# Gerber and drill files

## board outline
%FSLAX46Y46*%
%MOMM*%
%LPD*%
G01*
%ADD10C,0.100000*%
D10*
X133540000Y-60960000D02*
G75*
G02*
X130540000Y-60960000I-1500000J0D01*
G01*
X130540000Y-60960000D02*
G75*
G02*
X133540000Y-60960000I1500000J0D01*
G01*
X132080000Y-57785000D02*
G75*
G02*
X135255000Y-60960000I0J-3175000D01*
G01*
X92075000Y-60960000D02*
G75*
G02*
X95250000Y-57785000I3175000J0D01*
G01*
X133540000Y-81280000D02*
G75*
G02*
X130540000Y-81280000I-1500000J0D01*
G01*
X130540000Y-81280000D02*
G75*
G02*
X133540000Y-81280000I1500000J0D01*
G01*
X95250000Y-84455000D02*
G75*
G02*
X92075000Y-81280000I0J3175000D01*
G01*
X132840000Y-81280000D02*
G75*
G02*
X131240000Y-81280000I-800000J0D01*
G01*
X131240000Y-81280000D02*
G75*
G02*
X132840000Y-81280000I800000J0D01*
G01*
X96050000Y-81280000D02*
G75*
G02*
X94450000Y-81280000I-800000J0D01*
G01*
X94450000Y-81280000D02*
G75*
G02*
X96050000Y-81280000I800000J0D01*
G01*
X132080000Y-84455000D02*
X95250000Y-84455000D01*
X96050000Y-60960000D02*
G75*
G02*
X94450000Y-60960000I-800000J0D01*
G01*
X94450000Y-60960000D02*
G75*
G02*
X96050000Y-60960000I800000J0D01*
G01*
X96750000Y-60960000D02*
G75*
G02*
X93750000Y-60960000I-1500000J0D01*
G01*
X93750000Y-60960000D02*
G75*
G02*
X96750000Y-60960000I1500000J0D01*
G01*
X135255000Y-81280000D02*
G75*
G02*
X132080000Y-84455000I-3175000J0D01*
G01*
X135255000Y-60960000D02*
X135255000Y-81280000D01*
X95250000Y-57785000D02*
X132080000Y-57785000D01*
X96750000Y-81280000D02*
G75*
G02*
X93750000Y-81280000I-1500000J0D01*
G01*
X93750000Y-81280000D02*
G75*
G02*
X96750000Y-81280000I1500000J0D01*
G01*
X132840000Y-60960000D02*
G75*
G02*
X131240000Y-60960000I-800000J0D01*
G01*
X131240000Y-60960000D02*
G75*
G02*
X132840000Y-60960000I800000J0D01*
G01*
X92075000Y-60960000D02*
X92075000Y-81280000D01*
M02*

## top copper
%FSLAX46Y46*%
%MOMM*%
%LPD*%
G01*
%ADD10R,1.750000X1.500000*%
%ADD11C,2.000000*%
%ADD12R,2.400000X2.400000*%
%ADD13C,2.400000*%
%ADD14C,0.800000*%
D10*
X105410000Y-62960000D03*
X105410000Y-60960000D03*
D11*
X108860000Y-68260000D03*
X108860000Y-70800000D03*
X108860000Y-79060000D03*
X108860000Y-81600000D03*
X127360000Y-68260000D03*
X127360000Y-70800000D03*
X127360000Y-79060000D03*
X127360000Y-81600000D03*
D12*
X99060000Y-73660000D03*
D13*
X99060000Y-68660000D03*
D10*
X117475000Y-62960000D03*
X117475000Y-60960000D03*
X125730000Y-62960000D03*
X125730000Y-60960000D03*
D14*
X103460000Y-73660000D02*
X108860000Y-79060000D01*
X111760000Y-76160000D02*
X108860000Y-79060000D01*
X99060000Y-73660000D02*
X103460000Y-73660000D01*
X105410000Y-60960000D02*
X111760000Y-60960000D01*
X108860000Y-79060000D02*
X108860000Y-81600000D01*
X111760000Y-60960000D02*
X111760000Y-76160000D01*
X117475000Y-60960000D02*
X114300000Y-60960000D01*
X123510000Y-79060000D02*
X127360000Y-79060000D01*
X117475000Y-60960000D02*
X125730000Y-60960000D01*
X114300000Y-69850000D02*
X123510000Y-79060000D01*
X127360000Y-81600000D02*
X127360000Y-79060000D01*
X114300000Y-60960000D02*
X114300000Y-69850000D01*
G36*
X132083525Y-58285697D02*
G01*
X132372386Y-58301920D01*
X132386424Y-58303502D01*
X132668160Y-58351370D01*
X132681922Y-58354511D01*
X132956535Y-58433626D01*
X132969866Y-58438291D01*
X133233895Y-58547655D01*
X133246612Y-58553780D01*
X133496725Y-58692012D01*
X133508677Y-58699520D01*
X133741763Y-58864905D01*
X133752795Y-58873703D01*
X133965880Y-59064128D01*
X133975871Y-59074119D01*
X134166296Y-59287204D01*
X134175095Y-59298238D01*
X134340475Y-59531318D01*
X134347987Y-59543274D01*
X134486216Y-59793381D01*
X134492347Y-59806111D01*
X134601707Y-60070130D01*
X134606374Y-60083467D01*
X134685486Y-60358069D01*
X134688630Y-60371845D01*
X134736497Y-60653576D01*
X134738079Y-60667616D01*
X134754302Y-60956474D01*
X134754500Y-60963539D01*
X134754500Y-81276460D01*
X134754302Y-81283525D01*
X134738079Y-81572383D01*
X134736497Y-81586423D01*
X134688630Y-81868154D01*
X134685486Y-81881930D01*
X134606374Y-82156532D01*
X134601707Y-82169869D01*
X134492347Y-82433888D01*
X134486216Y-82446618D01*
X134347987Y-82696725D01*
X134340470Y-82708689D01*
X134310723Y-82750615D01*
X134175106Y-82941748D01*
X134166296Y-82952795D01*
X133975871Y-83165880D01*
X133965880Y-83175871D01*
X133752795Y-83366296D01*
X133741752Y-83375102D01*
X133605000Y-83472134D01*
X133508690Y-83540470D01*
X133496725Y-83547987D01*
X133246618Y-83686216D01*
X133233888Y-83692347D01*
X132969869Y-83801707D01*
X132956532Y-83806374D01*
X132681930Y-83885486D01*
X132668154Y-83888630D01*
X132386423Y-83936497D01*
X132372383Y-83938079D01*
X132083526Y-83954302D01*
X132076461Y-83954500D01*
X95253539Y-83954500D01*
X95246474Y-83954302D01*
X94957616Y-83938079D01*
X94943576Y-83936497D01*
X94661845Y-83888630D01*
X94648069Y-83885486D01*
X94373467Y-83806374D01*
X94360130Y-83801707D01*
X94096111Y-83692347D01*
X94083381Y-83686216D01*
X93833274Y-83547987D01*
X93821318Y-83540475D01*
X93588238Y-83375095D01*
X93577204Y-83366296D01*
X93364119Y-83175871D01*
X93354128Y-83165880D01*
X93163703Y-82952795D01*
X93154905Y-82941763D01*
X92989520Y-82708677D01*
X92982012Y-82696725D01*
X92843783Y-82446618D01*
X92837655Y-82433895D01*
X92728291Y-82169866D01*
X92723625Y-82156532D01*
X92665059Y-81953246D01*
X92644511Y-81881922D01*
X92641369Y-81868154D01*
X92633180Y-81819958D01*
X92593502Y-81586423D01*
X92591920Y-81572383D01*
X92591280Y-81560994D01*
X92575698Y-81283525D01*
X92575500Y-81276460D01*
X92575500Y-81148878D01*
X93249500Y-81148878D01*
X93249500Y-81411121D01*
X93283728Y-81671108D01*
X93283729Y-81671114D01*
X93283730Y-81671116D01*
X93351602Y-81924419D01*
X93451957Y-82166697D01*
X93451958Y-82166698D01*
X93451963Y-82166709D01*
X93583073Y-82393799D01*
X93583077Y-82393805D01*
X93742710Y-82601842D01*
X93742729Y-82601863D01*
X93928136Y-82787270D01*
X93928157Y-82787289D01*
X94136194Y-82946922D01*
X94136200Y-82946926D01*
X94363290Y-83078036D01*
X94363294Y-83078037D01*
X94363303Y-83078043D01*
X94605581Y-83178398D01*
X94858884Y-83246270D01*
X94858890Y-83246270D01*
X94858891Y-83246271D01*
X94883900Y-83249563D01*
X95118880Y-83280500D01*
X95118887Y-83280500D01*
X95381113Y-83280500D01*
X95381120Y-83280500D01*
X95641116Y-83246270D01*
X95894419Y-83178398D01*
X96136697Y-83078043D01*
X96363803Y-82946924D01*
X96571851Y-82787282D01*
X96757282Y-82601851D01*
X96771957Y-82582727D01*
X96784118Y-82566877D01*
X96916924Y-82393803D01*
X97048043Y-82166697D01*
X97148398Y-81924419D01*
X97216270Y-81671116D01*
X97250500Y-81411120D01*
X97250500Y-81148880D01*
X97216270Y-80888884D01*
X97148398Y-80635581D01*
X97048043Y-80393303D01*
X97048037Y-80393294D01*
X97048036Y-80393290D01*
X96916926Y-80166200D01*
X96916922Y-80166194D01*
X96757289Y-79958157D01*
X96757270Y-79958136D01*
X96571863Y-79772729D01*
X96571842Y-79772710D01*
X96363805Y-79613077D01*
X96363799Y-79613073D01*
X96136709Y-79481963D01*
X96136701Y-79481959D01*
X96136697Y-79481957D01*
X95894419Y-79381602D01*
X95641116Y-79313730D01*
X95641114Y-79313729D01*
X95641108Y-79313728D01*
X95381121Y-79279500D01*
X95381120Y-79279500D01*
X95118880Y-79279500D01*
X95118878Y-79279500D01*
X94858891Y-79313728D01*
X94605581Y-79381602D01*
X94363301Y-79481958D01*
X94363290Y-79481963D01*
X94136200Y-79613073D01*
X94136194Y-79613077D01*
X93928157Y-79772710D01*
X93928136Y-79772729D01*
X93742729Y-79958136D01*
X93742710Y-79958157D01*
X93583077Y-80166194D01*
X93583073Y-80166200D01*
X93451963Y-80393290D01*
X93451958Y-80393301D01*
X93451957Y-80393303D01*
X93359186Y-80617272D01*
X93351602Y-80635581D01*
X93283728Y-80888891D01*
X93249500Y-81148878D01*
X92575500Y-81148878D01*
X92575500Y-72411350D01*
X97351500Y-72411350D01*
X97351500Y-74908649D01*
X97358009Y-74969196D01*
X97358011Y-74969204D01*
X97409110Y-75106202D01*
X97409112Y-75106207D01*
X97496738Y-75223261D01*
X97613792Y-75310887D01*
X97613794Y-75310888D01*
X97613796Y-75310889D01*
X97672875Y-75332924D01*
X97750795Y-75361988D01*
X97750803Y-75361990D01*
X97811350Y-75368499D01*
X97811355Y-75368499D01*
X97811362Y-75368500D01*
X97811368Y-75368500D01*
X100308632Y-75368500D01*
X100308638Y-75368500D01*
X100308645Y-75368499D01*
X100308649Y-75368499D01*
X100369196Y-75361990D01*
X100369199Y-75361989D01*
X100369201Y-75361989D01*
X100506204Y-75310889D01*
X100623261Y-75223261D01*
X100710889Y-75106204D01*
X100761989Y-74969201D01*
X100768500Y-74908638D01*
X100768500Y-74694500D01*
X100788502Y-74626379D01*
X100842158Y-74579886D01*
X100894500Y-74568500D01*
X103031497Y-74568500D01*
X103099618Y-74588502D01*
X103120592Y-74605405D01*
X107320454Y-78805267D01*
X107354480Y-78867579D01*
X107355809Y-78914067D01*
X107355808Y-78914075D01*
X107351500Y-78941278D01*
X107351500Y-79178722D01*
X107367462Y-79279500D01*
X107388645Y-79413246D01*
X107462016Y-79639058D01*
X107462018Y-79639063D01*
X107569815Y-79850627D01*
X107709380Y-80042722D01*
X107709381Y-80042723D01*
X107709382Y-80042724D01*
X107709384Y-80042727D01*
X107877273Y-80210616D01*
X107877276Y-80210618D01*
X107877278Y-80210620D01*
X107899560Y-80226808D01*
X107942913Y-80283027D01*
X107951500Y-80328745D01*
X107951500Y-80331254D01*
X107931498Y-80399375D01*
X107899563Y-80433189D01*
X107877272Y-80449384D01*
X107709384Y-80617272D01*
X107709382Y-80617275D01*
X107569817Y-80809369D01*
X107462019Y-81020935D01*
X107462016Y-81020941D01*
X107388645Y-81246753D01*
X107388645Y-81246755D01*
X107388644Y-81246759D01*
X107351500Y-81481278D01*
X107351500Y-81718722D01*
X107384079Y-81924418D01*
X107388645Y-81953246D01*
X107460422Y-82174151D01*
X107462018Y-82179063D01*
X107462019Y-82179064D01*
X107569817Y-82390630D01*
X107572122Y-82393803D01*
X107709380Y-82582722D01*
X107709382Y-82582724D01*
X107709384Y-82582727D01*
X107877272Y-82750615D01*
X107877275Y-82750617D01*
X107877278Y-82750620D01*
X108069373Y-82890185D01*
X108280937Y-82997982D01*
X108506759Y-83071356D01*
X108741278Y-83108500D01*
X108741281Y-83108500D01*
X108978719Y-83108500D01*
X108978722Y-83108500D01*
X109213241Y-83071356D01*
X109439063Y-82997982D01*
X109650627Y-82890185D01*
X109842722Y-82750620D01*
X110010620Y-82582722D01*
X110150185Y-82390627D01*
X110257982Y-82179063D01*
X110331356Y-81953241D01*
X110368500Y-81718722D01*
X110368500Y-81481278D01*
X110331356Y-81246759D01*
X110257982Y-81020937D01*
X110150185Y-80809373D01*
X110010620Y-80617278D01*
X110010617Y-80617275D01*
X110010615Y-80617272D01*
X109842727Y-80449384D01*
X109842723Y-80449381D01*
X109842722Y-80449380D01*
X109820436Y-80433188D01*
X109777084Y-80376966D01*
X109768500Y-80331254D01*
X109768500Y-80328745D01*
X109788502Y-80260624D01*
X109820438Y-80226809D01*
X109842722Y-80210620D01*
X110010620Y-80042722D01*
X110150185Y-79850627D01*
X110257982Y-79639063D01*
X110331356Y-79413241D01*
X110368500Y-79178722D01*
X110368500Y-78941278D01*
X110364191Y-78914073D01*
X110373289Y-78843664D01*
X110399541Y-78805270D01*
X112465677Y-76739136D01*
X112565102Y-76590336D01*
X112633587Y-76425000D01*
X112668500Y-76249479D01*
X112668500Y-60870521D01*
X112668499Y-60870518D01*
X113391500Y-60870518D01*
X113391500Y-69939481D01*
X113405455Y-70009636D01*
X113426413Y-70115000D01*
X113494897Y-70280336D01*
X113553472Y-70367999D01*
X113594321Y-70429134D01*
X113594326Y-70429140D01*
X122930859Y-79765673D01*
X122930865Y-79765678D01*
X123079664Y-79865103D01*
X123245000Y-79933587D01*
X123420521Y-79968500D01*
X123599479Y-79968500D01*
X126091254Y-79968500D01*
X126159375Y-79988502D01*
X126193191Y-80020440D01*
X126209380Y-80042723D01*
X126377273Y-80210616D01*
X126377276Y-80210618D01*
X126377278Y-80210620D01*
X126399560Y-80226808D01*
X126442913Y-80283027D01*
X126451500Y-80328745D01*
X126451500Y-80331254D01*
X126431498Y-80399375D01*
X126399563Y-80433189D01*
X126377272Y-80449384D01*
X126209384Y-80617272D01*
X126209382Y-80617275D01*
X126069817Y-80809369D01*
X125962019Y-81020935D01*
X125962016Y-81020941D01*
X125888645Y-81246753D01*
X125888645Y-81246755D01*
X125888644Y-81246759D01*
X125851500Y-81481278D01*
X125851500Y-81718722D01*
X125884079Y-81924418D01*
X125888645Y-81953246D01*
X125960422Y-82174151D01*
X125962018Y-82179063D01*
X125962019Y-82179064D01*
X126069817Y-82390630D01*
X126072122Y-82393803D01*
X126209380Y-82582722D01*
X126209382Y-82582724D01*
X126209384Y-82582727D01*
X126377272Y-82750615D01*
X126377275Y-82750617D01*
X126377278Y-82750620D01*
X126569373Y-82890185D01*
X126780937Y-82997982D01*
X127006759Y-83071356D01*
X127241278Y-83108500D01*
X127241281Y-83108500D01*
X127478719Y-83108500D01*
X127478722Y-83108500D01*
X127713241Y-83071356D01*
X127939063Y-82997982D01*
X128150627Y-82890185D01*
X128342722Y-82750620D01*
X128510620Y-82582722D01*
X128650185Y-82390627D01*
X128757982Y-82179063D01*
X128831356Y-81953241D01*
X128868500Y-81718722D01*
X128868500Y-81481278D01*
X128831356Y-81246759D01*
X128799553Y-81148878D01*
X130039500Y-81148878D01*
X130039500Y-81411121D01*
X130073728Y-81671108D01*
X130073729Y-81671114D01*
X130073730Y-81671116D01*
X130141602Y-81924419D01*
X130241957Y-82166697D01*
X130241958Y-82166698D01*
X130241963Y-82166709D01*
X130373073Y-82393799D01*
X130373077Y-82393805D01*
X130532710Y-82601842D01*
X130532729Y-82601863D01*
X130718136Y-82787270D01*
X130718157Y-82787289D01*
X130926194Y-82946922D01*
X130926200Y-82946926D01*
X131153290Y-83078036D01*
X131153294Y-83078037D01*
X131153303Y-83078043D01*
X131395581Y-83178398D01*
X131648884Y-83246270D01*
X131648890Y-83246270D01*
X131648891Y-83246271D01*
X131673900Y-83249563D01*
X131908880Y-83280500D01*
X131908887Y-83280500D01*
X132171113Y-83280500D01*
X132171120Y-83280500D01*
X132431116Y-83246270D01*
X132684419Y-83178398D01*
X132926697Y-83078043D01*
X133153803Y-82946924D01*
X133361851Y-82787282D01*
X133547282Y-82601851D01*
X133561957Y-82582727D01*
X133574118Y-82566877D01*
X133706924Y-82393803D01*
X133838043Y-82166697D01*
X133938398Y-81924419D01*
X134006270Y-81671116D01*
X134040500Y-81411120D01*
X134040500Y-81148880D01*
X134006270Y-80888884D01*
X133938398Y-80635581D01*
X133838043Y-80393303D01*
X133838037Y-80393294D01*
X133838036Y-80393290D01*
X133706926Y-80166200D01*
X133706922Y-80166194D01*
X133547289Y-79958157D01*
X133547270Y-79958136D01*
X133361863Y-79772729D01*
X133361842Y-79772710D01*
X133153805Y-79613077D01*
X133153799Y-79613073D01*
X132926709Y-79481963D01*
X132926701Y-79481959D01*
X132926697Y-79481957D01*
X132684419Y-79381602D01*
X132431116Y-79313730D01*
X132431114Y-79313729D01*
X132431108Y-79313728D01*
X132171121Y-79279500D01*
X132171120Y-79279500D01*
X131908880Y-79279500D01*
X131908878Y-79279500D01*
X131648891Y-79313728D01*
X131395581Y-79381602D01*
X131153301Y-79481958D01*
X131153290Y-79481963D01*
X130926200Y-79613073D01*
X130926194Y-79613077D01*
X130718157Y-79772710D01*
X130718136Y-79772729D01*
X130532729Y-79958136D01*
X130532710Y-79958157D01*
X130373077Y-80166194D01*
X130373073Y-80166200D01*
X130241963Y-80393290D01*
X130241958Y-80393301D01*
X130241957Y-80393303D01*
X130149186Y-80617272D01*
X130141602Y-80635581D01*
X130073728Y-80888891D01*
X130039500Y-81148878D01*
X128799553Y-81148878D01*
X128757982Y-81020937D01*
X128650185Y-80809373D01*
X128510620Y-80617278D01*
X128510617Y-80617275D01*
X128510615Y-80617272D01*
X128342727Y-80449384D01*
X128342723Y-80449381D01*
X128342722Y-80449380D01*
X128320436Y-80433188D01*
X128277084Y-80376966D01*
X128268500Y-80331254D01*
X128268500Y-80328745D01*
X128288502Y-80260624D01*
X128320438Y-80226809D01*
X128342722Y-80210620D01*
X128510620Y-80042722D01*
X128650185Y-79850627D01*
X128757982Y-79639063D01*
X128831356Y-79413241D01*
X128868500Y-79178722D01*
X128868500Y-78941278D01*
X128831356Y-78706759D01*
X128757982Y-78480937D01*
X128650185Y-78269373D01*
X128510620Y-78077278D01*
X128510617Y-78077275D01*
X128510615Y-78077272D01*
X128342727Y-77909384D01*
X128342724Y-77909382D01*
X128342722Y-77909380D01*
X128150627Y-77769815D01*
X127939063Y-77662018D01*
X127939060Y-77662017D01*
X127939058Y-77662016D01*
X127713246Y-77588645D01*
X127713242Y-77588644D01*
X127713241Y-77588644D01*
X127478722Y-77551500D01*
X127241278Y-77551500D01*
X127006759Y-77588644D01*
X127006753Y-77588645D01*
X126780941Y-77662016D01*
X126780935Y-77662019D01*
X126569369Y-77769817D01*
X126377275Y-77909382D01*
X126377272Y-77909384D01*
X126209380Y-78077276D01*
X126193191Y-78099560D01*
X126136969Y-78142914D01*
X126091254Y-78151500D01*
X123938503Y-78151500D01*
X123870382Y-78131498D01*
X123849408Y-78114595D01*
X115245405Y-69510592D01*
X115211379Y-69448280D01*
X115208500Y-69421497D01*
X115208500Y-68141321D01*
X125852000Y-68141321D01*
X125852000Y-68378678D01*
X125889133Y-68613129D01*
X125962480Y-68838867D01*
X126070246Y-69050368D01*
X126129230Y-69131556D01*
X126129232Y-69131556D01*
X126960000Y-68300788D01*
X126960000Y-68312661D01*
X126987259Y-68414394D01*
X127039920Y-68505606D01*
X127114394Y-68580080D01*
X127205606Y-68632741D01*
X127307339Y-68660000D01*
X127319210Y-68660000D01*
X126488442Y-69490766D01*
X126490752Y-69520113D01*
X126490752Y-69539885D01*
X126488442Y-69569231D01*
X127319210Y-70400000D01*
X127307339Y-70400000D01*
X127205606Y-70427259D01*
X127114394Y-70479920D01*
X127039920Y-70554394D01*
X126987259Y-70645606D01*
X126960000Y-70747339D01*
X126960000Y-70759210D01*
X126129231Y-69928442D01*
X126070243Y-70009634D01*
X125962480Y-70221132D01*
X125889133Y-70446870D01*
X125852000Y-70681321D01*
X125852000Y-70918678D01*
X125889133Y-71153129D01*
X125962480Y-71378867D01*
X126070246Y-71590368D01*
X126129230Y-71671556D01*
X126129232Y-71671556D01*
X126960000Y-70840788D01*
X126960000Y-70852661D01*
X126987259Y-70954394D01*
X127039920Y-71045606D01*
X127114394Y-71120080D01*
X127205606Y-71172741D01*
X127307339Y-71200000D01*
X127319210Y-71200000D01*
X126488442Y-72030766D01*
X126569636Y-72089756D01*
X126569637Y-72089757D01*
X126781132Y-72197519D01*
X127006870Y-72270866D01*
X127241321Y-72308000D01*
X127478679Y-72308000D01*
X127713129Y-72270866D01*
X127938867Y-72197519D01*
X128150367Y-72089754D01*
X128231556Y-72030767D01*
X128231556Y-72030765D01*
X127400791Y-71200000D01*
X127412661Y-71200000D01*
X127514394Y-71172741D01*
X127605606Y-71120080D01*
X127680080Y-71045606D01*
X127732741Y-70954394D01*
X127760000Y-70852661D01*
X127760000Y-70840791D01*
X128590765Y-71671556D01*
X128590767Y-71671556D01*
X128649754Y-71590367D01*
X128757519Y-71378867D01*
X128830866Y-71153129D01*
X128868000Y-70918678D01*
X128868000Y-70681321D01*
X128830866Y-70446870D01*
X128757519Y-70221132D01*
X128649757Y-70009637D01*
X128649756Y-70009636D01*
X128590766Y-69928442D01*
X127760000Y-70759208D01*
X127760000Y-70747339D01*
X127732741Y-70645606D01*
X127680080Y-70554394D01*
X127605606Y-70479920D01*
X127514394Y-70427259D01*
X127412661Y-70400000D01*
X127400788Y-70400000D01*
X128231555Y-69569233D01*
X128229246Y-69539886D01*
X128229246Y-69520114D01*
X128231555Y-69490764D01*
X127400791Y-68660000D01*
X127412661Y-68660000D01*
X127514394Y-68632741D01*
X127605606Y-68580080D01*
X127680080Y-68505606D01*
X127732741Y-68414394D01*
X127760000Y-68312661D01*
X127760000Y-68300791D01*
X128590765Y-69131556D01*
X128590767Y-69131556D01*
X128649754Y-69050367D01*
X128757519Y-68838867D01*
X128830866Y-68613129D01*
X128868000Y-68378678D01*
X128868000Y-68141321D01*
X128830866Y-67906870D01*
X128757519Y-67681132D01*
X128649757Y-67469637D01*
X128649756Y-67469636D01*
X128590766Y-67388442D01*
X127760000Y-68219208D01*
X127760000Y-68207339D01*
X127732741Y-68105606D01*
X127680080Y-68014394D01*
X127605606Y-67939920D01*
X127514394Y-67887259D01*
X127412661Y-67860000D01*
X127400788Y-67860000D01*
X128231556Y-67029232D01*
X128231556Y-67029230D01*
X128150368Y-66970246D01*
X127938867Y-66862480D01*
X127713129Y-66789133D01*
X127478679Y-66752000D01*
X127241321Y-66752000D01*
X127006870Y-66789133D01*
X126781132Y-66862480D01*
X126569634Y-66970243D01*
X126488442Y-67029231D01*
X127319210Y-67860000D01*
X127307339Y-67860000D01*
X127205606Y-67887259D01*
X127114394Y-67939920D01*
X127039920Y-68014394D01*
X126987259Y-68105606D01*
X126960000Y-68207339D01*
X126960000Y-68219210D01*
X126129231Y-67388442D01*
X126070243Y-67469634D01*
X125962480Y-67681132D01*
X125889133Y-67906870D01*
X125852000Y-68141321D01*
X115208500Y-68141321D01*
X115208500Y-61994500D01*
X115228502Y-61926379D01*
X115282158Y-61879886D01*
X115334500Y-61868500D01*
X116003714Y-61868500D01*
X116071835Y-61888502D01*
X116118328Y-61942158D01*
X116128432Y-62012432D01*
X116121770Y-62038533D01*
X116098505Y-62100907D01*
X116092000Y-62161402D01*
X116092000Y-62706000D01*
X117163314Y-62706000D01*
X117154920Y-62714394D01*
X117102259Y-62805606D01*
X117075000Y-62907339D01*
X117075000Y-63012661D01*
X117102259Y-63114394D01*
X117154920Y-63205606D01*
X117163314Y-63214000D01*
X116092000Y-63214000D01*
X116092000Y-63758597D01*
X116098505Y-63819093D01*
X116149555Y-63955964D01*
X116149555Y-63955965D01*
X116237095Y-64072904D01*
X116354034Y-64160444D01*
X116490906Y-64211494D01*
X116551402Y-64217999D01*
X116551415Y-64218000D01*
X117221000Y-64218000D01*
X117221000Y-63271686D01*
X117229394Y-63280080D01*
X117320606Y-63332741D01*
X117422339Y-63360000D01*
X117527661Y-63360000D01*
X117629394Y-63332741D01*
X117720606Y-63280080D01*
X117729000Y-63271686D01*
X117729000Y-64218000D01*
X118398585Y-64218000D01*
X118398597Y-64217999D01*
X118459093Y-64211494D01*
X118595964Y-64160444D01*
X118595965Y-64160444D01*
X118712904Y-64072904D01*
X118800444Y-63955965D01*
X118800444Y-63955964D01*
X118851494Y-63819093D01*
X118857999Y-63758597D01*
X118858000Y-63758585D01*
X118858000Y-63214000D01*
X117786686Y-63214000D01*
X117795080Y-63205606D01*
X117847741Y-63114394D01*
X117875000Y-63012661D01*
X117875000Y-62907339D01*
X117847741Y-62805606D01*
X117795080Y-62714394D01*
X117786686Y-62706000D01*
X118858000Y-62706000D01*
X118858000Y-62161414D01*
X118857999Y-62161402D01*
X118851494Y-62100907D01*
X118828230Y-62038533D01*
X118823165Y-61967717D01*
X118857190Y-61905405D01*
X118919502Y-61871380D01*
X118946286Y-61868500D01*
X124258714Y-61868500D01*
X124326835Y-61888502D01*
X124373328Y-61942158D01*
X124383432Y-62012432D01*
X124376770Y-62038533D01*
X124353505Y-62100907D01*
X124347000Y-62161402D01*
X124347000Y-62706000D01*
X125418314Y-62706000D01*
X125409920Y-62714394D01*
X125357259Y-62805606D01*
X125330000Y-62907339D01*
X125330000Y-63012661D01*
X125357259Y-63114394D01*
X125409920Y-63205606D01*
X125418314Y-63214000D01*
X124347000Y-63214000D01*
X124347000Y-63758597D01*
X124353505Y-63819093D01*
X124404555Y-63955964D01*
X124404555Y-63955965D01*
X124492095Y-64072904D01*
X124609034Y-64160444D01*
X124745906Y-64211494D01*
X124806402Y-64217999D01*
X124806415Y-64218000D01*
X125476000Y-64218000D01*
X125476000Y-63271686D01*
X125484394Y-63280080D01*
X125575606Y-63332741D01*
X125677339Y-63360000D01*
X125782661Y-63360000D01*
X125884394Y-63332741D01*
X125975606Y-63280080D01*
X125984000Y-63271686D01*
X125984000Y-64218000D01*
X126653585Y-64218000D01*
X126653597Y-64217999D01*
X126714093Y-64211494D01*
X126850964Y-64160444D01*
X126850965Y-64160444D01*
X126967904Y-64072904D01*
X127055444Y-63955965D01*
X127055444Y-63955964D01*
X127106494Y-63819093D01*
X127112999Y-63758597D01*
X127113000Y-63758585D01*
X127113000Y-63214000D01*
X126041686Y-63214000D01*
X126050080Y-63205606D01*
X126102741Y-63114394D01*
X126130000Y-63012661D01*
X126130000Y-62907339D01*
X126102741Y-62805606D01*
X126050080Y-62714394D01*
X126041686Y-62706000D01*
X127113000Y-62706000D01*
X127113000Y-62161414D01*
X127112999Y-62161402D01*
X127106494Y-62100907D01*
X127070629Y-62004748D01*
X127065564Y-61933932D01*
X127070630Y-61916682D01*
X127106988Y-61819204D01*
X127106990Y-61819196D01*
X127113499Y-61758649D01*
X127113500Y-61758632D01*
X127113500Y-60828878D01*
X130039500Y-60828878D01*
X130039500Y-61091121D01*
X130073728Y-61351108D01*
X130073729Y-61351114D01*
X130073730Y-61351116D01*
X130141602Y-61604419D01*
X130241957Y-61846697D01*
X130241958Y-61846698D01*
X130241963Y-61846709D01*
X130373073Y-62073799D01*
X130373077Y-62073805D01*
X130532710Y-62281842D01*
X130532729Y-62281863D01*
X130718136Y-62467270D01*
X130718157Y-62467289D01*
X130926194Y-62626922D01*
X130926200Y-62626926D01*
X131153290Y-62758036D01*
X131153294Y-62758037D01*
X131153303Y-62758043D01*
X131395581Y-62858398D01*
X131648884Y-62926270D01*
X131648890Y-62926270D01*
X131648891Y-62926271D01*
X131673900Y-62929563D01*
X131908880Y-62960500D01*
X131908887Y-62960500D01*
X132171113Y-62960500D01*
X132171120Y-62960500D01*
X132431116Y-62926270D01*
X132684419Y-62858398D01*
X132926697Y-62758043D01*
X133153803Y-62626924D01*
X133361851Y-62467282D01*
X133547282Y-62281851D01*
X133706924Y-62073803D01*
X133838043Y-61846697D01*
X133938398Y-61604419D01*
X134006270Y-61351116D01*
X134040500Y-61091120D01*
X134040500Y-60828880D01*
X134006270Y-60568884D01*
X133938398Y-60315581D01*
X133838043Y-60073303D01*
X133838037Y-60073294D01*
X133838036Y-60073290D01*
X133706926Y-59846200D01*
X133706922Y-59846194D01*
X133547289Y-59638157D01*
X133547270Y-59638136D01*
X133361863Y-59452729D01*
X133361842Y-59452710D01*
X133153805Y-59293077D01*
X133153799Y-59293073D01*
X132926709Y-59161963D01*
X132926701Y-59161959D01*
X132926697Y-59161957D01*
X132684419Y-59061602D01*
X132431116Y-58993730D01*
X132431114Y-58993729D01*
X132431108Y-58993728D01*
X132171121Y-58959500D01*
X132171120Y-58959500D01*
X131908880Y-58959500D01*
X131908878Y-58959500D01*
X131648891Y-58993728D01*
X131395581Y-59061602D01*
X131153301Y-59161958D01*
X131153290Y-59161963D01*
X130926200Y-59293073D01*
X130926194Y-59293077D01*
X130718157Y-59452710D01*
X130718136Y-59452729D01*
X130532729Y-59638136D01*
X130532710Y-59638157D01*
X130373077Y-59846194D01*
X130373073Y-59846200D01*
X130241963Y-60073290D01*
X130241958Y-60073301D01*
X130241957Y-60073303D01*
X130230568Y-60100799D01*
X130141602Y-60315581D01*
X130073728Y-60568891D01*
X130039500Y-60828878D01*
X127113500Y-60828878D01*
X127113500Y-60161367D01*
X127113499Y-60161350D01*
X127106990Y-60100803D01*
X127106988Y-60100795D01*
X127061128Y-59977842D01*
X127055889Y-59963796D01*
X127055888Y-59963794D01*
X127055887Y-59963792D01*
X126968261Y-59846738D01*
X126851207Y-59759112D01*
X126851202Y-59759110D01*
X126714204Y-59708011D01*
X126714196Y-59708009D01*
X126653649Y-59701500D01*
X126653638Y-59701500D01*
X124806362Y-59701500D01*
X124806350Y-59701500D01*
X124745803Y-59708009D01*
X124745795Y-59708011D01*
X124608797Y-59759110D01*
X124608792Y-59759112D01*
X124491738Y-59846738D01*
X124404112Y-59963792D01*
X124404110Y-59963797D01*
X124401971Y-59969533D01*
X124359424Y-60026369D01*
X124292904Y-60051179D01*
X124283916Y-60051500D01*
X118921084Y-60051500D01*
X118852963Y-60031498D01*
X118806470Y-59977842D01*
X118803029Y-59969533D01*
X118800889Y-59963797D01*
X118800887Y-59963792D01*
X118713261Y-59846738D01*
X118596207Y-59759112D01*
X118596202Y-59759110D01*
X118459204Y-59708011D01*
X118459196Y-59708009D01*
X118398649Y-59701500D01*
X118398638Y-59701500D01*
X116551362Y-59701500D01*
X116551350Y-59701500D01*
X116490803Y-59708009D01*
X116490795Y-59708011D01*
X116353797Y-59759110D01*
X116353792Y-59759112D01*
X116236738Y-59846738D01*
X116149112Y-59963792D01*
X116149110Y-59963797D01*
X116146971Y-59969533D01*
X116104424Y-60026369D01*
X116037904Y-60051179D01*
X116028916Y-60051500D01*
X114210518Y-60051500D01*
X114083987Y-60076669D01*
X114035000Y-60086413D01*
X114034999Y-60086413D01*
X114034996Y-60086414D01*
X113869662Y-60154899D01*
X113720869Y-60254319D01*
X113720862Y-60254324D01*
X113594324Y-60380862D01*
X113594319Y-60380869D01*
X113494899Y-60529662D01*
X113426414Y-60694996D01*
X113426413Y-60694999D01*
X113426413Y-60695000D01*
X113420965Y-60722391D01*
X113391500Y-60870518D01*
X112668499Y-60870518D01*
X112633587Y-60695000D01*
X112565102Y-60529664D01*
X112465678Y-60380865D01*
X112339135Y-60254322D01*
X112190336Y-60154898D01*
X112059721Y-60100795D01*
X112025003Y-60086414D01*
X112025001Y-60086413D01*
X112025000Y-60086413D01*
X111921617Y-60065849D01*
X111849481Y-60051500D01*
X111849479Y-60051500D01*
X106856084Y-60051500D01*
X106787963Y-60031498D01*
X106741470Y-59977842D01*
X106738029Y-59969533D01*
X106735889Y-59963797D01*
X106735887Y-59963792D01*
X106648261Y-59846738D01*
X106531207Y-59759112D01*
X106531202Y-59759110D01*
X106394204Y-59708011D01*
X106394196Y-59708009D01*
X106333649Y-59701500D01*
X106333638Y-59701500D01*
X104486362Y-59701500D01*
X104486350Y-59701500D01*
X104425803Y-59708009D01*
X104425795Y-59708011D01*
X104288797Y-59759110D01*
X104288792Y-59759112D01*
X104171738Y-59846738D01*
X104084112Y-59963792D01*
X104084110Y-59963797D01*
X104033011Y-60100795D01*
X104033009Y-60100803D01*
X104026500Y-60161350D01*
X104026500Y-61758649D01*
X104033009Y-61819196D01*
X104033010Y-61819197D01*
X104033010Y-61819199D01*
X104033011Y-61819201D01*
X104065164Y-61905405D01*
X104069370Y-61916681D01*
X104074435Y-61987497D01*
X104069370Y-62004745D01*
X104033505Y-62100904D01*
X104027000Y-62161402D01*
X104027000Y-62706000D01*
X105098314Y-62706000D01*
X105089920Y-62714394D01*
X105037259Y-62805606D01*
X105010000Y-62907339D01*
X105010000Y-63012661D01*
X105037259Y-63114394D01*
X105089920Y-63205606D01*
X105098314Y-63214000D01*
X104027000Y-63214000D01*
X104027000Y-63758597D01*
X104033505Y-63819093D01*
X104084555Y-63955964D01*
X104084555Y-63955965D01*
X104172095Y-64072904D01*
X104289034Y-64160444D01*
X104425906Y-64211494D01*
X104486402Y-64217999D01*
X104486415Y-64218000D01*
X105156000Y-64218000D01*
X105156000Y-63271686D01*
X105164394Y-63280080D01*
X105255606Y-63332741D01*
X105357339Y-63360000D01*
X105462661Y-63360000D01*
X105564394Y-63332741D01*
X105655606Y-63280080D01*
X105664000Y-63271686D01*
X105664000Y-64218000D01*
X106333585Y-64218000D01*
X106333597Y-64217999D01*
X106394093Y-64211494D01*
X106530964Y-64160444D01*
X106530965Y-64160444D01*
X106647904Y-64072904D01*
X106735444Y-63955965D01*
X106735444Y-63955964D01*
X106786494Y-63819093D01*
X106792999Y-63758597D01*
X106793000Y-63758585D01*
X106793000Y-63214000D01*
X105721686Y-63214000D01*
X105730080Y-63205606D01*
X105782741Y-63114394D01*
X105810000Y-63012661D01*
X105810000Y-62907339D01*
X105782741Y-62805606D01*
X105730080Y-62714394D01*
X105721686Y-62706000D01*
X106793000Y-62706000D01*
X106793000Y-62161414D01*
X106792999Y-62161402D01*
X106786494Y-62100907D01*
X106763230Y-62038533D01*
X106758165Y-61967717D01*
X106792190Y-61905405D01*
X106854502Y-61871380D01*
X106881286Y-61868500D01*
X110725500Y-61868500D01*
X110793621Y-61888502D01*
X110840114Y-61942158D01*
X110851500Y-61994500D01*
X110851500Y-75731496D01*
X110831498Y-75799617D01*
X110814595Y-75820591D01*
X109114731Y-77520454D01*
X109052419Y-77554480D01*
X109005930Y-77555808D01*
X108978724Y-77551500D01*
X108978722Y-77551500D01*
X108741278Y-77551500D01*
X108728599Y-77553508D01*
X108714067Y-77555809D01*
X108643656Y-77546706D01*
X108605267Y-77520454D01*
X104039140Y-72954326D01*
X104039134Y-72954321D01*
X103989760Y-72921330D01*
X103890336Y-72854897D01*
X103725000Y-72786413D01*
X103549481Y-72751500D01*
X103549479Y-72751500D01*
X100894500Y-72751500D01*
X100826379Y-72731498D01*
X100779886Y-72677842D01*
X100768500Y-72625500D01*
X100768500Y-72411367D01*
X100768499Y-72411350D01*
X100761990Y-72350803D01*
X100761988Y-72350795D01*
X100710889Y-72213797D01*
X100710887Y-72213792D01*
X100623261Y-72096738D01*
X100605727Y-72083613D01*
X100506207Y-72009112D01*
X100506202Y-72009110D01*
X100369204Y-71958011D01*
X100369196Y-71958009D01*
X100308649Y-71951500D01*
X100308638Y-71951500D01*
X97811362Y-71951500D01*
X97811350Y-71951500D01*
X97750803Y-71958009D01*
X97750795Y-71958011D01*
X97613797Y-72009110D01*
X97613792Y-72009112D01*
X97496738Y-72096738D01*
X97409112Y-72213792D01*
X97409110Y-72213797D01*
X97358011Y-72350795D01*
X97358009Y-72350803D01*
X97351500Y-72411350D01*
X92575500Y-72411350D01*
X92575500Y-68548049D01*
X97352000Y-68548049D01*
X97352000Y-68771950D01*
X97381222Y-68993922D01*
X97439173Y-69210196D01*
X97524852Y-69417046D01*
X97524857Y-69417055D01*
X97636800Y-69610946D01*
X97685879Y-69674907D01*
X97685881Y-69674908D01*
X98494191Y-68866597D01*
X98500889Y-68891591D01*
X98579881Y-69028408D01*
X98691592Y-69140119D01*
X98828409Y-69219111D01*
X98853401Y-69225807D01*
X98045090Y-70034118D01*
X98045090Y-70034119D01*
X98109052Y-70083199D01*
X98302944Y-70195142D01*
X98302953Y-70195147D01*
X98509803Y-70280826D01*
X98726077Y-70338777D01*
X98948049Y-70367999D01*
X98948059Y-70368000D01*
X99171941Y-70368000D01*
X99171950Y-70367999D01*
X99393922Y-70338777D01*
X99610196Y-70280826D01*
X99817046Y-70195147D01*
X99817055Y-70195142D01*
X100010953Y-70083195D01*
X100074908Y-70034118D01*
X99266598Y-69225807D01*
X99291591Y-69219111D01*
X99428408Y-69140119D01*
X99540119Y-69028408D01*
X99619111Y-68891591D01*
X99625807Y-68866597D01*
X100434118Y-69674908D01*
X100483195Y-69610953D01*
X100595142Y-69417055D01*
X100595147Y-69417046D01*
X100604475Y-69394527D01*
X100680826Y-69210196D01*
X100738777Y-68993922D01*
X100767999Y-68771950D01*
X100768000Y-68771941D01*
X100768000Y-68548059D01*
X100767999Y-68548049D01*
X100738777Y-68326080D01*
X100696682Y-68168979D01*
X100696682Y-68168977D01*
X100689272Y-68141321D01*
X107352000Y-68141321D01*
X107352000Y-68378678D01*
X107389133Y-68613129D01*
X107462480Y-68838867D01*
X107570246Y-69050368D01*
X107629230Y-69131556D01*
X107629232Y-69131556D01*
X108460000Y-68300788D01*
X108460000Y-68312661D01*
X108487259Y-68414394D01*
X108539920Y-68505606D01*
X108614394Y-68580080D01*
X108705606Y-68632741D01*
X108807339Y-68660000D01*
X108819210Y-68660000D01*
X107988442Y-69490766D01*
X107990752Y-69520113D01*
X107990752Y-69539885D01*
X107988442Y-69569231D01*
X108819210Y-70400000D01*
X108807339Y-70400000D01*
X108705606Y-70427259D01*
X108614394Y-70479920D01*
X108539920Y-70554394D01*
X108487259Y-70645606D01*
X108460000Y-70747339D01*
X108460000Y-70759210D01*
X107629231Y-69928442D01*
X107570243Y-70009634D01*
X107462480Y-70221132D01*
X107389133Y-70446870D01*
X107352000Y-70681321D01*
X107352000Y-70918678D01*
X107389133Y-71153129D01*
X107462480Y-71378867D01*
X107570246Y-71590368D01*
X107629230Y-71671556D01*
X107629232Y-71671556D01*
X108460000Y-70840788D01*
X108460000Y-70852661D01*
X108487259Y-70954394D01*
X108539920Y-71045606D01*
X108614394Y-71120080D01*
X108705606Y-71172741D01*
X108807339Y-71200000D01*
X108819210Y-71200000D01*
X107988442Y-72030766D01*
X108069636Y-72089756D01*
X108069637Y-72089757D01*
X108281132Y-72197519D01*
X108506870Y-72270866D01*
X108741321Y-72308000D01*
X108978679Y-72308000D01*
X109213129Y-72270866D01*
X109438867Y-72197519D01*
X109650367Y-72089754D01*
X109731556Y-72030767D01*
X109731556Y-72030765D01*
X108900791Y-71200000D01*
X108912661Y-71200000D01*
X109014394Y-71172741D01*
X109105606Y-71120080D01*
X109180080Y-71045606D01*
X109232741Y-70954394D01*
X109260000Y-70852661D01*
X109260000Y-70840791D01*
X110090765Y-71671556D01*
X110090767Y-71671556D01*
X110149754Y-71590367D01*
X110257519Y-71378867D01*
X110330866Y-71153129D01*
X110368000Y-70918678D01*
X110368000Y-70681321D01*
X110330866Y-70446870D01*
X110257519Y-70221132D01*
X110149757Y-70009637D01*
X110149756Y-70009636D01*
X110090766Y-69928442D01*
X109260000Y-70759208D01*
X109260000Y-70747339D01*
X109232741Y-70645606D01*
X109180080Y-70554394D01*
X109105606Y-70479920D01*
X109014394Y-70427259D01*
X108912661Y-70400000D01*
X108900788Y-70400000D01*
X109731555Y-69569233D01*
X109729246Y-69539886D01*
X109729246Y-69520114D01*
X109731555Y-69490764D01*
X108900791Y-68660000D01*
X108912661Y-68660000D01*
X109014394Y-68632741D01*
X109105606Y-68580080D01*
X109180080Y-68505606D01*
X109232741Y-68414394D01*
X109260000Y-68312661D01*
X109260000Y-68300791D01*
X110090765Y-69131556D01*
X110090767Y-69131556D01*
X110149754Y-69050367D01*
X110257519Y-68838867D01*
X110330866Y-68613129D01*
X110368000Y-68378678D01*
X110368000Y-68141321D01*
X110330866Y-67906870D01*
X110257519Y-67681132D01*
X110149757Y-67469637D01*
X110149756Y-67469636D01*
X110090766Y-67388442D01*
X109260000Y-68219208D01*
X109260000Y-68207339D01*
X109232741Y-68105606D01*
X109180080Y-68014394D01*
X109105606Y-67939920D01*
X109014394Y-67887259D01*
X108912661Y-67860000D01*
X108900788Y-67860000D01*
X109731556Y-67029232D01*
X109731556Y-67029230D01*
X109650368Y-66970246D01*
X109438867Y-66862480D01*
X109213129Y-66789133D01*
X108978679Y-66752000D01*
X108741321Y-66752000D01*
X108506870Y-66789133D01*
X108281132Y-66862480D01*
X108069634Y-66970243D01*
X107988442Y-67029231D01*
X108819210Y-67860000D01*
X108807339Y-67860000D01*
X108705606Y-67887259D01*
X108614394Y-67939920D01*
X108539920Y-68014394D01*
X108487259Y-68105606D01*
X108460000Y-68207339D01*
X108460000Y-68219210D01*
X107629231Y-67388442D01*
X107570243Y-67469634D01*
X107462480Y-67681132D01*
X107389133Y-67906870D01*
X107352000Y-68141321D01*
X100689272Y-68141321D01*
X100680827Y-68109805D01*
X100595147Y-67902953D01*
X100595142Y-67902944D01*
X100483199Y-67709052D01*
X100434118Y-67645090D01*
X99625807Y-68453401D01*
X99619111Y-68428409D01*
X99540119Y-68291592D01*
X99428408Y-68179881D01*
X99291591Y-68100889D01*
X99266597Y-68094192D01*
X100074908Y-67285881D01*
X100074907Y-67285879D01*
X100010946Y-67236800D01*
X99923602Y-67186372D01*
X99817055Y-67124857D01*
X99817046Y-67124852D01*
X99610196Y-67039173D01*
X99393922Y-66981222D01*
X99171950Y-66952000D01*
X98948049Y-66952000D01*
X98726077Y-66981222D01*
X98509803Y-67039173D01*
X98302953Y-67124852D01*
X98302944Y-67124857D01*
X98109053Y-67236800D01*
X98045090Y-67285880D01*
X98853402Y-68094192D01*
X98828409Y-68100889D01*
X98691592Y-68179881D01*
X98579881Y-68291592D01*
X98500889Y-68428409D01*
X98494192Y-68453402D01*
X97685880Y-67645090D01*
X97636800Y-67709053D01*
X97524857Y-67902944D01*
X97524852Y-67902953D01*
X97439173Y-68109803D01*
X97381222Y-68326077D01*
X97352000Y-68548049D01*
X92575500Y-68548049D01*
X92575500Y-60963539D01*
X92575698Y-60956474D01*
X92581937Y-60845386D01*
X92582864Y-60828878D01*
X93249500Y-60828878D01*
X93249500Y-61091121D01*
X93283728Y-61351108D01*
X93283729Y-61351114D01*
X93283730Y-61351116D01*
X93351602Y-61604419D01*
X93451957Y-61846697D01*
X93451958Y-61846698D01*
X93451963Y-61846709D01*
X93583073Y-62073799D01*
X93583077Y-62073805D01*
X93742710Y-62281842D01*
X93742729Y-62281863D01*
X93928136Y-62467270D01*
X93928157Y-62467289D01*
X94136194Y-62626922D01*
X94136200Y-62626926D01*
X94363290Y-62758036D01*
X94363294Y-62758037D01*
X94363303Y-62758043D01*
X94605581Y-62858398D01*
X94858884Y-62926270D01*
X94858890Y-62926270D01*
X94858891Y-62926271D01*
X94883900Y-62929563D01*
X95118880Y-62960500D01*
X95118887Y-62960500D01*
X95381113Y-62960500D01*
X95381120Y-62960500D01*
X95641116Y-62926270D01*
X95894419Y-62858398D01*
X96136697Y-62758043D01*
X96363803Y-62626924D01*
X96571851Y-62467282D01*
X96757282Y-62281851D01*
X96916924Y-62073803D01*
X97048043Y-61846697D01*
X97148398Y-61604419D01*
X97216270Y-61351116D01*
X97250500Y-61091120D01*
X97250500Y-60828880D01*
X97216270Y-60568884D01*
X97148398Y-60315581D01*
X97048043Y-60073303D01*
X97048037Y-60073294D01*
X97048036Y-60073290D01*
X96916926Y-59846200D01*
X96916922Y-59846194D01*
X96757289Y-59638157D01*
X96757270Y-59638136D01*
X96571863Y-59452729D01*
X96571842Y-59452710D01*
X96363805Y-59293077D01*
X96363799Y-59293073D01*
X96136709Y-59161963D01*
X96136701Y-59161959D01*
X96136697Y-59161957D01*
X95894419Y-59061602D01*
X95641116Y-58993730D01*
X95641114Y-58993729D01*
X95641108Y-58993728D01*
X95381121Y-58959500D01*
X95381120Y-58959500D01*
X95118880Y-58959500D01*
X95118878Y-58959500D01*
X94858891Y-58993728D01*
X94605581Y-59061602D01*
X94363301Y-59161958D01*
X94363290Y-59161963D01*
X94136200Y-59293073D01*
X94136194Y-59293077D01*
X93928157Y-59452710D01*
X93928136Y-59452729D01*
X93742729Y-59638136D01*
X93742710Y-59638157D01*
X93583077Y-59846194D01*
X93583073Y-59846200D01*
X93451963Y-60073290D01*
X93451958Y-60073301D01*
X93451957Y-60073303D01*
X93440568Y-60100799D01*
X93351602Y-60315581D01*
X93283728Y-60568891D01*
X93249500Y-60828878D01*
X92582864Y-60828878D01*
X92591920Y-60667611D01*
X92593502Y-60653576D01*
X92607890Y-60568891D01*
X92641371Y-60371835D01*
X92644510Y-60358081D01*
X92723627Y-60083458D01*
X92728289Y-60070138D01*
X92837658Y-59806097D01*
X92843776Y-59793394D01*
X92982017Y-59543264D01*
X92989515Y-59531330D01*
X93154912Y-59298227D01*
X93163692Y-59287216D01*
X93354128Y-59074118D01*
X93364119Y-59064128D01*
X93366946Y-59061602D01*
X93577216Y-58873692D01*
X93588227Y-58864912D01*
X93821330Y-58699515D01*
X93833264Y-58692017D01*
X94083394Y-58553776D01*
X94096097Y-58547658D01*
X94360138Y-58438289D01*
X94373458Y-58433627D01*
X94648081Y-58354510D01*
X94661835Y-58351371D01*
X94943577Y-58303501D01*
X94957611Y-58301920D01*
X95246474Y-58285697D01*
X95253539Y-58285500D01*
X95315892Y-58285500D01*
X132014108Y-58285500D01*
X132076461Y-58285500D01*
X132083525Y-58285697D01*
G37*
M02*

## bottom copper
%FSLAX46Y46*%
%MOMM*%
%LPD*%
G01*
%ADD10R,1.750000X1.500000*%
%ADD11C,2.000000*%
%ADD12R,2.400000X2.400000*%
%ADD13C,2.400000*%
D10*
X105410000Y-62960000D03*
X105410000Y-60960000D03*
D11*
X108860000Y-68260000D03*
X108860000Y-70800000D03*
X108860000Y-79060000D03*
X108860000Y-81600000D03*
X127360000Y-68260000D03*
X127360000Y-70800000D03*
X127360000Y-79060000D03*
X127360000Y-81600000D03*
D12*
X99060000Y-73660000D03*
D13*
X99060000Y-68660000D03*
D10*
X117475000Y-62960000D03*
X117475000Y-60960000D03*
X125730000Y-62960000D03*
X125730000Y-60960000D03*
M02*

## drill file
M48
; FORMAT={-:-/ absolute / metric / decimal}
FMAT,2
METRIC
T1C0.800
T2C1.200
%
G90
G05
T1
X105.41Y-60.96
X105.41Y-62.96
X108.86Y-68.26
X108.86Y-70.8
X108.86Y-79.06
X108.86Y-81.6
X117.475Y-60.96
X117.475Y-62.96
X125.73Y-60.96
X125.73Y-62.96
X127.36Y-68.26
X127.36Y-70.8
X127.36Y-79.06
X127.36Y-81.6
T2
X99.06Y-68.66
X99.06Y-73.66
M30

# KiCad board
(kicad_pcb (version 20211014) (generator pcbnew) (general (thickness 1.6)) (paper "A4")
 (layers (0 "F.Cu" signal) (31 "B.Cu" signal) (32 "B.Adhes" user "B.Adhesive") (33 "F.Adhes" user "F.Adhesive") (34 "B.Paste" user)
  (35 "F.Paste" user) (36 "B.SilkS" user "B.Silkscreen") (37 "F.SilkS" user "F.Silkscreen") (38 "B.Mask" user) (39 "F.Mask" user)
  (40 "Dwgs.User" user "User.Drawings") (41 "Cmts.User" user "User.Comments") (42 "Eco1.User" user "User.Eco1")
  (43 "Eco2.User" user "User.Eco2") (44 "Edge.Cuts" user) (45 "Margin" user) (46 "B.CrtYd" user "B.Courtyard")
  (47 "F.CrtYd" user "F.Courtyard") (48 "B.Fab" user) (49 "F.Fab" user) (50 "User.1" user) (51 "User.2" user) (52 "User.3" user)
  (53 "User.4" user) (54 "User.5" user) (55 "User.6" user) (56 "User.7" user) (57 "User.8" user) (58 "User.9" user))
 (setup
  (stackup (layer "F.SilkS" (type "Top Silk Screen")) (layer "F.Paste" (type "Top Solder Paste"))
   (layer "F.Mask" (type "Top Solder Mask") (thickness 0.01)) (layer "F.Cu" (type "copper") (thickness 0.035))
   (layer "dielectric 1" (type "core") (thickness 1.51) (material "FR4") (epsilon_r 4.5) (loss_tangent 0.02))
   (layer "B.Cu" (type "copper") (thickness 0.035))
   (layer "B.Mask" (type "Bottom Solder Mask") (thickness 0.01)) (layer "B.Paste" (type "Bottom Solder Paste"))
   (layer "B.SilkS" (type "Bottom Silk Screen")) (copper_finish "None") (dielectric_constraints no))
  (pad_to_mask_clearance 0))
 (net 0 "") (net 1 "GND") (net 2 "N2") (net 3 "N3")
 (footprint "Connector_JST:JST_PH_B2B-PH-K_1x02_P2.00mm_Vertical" (layer "F.Cu") (at 105.41 62.96 90)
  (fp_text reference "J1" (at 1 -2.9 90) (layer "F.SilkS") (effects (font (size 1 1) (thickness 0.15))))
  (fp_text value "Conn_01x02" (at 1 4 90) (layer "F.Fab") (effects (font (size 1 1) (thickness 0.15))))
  (pad "1" thru_hole rect (at 0 0 90) (size 1.5 1.75) (drill 0.8) (layers *.Cu *.Mask) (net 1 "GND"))
  (pad "2" thru_hole rect (at 2 0 90) (size 1.5 1.75) (drill 0.8) (layers *.Cu *.Mask) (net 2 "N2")))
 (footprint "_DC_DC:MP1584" (layer "F.Cu") (at 108.86 68.26)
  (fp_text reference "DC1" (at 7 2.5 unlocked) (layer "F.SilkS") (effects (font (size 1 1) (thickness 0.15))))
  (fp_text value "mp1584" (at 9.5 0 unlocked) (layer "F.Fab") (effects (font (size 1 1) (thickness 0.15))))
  (pad "1" thru_hole circle (at 0 0) (size 2 2) (drill 0.8) (layers *.Cu *.Mask) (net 1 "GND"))
  (pad "2" thru_hole circle (at 0 2.54) (size 2 2) (drill 0.8) (layers *.Cu *.Mask) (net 1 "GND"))
  (pad "3" thru_hole circle (at 0 10.8) (size 2 2) (drill 0.8) (layers *.Cu *.Mask) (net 2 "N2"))
  (pad "4" thru_hole circle (at 0 13.34) (size 2 2) (drill 0.8) (layers *.Cu *.Mask) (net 2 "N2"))
  (pad "5" thru_hole circle (at 18.5 0) (size 2 2) (drill 0.8) (layers *.Cu *.Mask) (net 1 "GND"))
  (pad "6" thru_hole circle (at 18.5 2.54) (size 2 2) (drill 0.8) (layers *.Cu *.Mask) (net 1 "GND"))
  (pad "7" thru_hole circle (at 18.5 10.8) (size 2 2) (drill 0.8) (layers *.Cu *.Mask) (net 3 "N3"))
  (pad "8" thru_hole circle (at 18.5 13.34) (size 2 2) (drill 0.8) (layers *.Cu *.Mask) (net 3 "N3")))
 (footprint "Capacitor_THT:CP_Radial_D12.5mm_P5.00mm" (layer "F.Cu") (at 99.06 73.66 90)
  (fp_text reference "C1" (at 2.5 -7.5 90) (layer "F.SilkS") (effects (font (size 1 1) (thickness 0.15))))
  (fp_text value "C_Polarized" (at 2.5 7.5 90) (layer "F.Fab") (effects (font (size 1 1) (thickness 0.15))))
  (pad "1" thru_hole rect (at 0 0 90) (size 2.4 2.4) (drill 1.2) (layers *.Cu *.Mask) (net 2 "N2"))
  (pad "2" thru_hole circle (at 5 0 90) (size 2.4 2.4) (drill 1.2) (layers *.Cu *.Mask) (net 1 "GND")))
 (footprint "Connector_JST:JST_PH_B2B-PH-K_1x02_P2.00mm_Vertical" (layer "F.Cu") (at 117.475 62.96 90)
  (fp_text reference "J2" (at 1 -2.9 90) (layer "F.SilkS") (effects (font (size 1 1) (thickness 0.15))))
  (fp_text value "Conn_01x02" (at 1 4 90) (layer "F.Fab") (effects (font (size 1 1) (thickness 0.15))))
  (pad "1" thru_hole rect (at 0 0 90) (size 1.5 1.75) (drill 0.8) (layers *.Cu *.Mask) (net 1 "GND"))
  (pad "2" thru_hole rect (at 2 0 90) (size 1.5 1.75) (drill 0.8) (layers *.Cu *.Mask) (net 3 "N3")))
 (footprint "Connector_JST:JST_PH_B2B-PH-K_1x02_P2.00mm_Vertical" (layer "F.Cu") (at 125.73 62.96 90)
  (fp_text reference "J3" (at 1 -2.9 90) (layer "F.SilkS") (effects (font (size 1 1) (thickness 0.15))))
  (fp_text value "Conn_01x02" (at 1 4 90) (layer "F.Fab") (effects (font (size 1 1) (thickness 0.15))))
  (pad "1" thru_hole rect (at 0 0 90) (size 1.5 1.75) (drill 0.8) (layers *.Cu *.Mask) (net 1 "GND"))
  (pad "2" thru_hole rect (at 2 0 90) (size 1.5 1.75) (drill 0.8) (layers *.Cu *.Mask) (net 3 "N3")))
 (gr_circle (center 132.04 60.96) (end 133.54 60.96) (layer "Edge.Cuts") (width 0.1) (fill none))
 (gr_arc (start 132.08 57.785) (mid 134.325064 58.714936) (end 135.255 60.96) (layer "Edge.Cuts") (width 0.1))
 (gr_arc (start 92.075 60.96) (mid 93.004936 58.714936) (end 95.25 57.785) (layer "Edge.Cuts") (width 0.1))
 (gr_circle (center 132.04 81.28) (end 133.54 81.28) (layer "Edge.Cuts") (width 0.1) (fill none))
 (gr_arc (start 95.25 84.455) (mid 93.004936 83.525064) (end 92.075 81.28) (layer "Edge.Cuts") (width 0.1))
 (gr_circle (center 132.04 81.28) (end 132.84 81.28) (layer "Edge.Cuts") (width 0.1) (fill none))
 (gr_circle (center 95.25 81.28) (end 96.05 81.28) (layer "Edge.Cuts") (width 0.1) (fill none))
 (gr_line (start 132.08 84.455) (end 95.25 84.455) (layer "Edge.Cuts") (width 0.1))
 (gr_circle (center 95.25 60.96) (end 96.05 60.96) (layer "Edge.Cuts") (width 0.1) (fill none))
 (gr_circle (center 95.25 60.96) (end 96.75 60.96) (layer "Edge.Cuts") (width 0.1) (fill none))
 (gr_arc (start 135.255 81.28) (mid 134.325064 83.525064) (end 132.08 84.455) (layer "Edge.Cuts") (width 0.1))
 (gr_line (start 135.255 60.96) (end 135.255 81.28) (layer "Edge.Cuts") (width 0.1))
 (gr_line (start 95.25 57.785) (end 132.08 57.785) (layer "Edge.Cuts") (width 0.1))
 (gr_circle (center 95.25 81.28) (end 96.75 81.28) (layer "Edge.Cuts") (width 0.1) (fill none))
 (gr_circle (center 132.04 60.96) (end 132.84 60.96) (layer "Edge.Cuts") (width 0.1) (fill none))
 (gr_line (start 92.075 60.96) (end 92.075 81.28) (layer "Edge.Cuts") (width 0.1))
 (segment (start 103.46 73.66) (end 108.86 79.06) (width 0.8) (layer "F.Cu") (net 2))
 (segment (start 111.76 76.16) (end 108.86 79.06) (width 0.8) (layer "F.Cu") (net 2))
 (segment (start 99.06 73.66) (end 103.46 73.66) (width 0.8) (layer "F.Cu") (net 2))
 (segment (start 105.41 60.96) (end 111.76 60.96) (width 0.8) (layer "F.Cu") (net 2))
 (segment (start 108.86 79.06) (end 108.86 81.6) (width 0.8) (layer "F.Cu") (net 2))
 (segment (start 111.76 60.96) (end 111.76 76.16) (width 0.8) (layer "F.Cu") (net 2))
 (segment (start 117.475 60.96) (end 114.3 60.96) (width 0.8) (layer "F.Cu") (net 3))
 (segment (start 123.51 79.06) (end 127.36 79.06) (width 0.8) (layer "F.Cu") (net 3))
 (segment (start 117.475 60.96) (end 125.73 60.96) (width 0.8) (layer "F.Cu") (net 3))
 (segment (start 114.3 69.85) (end 123.51 79.06) (width 0.8) (layer "F.Cu") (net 3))
 (segment (start 127.36 81.6) (end 127.36 79.06) (width 0.8) (layer "F.Cu") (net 3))
 (segment (start 114.3 60.96) (end 114.3 69.85) (width 0.8) (layer "F.Cu") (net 3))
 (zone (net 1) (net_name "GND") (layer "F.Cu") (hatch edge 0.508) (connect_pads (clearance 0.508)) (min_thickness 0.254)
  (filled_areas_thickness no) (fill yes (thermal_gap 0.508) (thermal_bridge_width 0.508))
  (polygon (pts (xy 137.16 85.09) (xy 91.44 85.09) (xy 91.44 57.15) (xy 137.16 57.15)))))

